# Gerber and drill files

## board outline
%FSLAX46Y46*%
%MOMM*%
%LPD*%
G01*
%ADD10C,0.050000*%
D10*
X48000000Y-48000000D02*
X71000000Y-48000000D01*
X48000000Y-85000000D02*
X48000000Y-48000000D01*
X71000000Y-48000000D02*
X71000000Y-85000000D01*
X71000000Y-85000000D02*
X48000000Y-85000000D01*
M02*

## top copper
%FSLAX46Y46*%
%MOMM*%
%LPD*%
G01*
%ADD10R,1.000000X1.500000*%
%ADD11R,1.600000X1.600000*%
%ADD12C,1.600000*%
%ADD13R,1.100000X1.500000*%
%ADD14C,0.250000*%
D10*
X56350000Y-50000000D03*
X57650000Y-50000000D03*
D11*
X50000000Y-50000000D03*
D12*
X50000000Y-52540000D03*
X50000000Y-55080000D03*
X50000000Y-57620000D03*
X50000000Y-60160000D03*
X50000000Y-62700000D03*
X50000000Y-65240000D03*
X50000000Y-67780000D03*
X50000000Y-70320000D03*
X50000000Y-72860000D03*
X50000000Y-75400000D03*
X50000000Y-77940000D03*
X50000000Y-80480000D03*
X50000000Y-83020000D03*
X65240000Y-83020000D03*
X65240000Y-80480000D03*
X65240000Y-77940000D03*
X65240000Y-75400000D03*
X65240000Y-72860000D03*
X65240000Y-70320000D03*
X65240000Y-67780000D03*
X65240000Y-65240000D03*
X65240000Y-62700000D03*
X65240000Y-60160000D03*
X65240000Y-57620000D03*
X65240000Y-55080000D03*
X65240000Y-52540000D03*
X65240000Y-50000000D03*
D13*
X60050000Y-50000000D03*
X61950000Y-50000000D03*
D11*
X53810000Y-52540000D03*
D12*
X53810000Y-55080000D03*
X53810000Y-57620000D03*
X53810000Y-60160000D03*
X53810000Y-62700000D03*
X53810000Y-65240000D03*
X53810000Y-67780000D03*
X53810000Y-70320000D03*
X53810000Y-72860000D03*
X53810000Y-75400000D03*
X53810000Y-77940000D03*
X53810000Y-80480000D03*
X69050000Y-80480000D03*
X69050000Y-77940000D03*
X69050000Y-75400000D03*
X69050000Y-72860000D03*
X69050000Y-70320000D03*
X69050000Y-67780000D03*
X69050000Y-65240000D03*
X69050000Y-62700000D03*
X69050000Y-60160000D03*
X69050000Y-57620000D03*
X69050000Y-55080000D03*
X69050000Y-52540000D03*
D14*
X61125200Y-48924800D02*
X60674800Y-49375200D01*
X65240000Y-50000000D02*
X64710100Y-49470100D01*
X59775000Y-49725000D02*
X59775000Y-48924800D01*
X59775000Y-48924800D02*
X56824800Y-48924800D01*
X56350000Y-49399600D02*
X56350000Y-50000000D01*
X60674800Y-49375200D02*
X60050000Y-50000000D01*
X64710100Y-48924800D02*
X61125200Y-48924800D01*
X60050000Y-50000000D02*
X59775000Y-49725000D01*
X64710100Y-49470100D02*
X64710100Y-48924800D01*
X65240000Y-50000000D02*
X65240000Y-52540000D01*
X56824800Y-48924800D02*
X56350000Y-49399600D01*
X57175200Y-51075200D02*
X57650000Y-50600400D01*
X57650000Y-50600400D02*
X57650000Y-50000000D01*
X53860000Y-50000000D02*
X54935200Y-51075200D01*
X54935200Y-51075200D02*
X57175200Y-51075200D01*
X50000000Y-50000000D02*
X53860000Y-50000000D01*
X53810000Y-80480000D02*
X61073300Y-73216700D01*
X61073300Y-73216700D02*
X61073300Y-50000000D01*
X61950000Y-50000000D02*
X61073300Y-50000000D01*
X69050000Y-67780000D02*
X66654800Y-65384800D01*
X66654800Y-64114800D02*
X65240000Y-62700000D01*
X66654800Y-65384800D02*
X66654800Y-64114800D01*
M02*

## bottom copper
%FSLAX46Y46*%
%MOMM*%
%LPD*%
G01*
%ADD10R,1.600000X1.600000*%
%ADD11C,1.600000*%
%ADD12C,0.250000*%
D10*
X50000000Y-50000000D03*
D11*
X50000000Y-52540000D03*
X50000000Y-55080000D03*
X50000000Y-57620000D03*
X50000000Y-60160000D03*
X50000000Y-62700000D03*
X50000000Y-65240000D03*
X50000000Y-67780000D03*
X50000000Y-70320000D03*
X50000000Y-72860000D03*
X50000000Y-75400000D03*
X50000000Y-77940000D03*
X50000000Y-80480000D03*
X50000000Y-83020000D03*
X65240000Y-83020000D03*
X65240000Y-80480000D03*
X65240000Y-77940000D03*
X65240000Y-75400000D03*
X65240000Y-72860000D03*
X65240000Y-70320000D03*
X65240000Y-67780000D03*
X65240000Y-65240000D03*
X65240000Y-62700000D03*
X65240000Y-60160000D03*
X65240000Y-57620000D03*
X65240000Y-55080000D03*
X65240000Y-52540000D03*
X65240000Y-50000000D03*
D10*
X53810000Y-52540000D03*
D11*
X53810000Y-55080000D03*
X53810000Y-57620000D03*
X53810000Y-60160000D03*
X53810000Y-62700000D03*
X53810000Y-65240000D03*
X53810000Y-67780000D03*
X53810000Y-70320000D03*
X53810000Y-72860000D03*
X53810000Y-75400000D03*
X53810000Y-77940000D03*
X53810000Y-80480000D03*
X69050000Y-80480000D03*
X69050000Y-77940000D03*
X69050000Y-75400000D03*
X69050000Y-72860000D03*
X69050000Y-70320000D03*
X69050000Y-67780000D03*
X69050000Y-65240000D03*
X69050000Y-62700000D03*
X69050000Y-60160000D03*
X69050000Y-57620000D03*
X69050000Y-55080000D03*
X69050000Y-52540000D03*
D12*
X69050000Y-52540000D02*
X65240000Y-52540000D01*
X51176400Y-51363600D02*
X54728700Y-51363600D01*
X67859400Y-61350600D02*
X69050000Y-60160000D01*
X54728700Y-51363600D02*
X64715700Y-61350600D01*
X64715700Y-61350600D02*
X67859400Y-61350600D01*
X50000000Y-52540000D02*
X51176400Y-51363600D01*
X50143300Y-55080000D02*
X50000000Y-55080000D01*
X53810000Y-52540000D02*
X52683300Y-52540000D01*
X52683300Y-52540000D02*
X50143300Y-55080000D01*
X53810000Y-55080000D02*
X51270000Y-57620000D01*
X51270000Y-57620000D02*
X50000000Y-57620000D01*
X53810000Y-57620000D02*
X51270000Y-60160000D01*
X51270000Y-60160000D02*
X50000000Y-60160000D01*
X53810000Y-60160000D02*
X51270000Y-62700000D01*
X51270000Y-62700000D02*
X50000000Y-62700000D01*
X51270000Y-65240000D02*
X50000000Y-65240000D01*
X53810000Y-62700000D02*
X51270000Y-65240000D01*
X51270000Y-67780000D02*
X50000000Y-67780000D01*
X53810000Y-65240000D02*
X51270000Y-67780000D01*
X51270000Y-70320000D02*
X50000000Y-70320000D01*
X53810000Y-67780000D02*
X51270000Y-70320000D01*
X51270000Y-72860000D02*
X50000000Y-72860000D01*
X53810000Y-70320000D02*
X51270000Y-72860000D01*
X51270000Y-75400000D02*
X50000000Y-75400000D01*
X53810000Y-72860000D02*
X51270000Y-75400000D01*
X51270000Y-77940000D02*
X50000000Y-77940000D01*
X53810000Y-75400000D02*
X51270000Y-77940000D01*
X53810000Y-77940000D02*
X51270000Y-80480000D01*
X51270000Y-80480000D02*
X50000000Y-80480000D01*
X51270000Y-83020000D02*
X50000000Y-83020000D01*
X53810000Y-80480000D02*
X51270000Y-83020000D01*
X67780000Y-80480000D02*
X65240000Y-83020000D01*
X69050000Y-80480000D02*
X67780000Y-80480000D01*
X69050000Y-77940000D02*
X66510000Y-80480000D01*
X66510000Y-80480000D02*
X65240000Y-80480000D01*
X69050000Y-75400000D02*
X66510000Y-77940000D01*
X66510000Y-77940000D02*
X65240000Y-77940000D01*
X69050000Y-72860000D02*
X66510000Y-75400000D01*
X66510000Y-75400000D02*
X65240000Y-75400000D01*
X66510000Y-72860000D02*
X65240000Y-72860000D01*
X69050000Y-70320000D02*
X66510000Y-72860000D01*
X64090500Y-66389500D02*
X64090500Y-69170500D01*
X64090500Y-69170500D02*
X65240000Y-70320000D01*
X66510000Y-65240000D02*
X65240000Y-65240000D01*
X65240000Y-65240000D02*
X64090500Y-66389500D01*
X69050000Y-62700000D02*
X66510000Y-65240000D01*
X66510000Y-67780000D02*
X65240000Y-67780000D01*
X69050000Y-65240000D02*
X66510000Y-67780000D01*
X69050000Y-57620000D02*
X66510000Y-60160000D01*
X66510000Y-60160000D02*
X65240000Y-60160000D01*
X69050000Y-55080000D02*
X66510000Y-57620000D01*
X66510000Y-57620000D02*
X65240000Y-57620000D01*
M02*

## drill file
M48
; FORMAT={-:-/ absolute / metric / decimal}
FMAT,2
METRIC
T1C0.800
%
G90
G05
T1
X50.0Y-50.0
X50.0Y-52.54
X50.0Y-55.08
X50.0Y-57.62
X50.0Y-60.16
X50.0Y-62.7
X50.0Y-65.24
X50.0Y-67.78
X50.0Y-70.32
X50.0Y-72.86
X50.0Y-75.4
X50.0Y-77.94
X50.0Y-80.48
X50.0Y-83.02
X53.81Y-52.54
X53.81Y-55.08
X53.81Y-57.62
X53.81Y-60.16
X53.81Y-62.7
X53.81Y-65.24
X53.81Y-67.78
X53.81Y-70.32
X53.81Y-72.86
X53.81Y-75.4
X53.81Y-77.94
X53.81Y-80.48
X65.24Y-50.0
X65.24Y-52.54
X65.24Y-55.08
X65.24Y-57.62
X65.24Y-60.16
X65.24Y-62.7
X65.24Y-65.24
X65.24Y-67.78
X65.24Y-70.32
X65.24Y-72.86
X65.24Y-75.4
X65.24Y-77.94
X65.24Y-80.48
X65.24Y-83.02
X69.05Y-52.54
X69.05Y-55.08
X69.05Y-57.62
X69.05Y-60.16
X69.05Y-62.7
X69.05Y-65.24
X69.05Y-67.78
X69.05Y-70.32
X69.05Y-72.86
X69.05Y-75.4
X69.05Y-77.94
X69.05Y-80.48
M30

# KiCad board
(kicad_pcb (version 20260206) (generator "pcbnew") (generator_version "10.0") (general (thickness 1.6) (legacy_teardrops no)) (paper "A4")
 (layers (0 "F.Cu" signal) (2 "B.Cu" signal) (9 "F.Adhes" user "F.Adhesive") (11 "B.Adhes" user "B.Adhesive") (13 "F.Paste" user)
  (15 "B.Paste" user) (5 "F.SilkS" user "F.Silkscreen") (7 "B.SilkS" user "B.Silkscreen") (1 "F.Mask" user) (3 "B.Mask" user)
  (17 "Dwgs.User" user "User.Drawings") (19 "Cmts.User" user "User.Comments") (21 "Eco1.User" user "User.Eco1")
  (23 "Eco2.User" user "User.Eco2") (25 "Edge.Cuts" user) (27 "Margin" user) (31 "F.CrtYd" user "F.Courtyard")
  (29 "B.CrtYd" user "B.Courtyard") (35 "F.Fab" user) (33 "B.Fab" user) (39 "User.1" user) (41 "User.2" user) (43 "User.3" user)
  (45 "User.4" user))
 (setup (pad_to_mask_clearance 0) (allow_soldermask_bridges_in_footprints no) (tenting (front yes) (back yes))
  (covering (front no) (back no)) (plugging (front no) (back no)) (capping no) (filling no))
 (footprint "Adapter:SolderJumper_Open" (layer "F.Cu") (at 57 50)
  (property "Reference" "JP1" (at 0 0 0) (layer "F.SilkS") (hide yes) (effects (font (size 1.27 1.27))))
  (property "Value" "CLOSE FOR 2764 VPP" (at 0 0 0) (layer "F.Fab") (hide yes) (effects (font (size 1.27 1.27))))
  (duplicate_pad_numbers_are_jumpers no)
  (pad "1" smd rect (at -0.65 0) (size 1 1.5) (layers "F.Cu" "F.Mask") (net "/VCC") (thermal_bridge_angle 45))
  (pad "2" smd rect (at 0.65 0) (size 1 1.5) (layers "F.Cu" "F.Mask") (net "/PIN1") (thermal_bridge_angle 45)))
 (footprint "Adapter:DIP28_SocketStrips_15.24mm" (layer "F.Cu") (at 50 50)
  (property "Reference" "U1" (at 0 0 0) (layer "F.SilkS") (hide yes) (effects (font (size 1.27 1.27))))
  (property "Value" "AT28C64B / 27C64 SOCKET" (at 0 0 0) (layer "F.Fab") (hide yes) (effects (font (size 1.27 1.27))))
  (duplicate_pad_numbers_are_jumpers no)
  (pad "1" thru_hole rect (at 0 0) (size 1.6 1.6) (drill 0.8) (layers "*.Cu" "*.Mask") (remove_unused_layers no) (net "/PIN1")
   (thermal_bridge_angle 45))
  (pad "2" thru_hole circle (at 0 2.54) (size 1.6 1.6) (drill 0.8) (layers "*.Cu" "*.Mask") (remove_unused_layers no) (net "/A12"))
  (pad "3" thru_hole circle (at 0 5.08) (size 1.6 1.6) (drill 0.8) (layers "*.Cu" "*.Mask") (remove_unused_layers no) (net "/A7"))
  (pad "4" thru_hole circle (at 0 7.62) (size 1.6 1.6) (drill 0.8) (layers "*.Cu" "*.Mask") (remove_unused_layers no) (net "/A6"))
  (pad "5" thru_hole circle (at 0 10.16) (size 1.6 1.6) (drill 0.8) (layers "*.Cu" "*.Mask") (remove_unused_layers no) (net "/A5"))
  (pad "6" thru_hole circle (at 0 12.7) (size 1.6 1.6) (drill 0.8) (layers "*.Cu" "*.Mask") (remove_unused_layers no) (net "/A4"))
  (pad "7" thru_hole circle (at 0 15.24) (size 1.6 1.6) (drill 0.8) (layers "*.Cu" "*.Mask") (remove_unused_layers no) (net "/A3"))
  (pad "8" thru_hole circle (at 0 17.78) (size 1.6 1.6) (drill 0.8) (layers "*.Cu" "*.Mask") (remove_unused_layers no) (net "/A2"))
  (pad "9" thru_hole circle (at 0 20.32) (size 1.6 1.6) (drill 0.8) (layers "*.Cu" "*.Mask") (remove_unused_layers no) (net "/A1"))
  (pad "10" thru_hole circle (at 0 22.86) (size 1.6 1.6) (drill 0.8) (layers "*.Cu" "*.Mask") (remove_unused_layers no) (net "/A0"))
  (pad "11" thru_hole circle (at 0 25.4) (size 1.6 1.6) (drill 0.8) (layers "*.Cu" "*.Mask") (remove_unused_layers no) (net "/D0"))
  (pad "12" thru_hole circle (at 0 27.94) (size 1.6 1.6) (drill 0.8) (layers "*.Cu" "*.Mask") (remove_unused_layers no) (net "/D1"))
  (pad "13" thru_hole circle (at 0 30.48) (size 1.6 1.6) (drill 0.8) (layers "*.Cu" "*.Mask") (remove_unused_layers no) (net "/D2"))
  (pad "14" thru_hole circle (at 0 33.02) (size 1.6 1.6) (drill 0.8) (layers "*.Cu" "*.Mask") (remove_unused_layers no) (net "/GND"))
  (pad "15" thru_hole circle (at 15.24 33.02) (size 1.6 1.6) (drill 0.8) (layers "*.Cu" "*.Mask") (remove_unused_layers no) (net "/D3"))
  (pad "16" thru_hole circle (at 15.24 30.48) (size 1.6 1.6) (drill 0.8) (layers "*.Cu" "*.Mask") (remove_unused_layers no) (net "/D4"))
  (pad "17" thru_hole circle (at 15.24 27.94) (size 1.6 1.6) (drill 0.8) (layers "*.Cu" "*.Mask") (remove_unused_layers no) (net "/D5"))
  (pad "18" thru_hole circle (at 15.24 25.4) (size 1.6 1.6) (drill 0.8) (layers "*.Cu" "*.Mask") (remove_unused_layers no) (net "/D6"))
  (pad "19" thru_hole circle (at 15.24 22.86) (size 1.6 1.6) (drill 0.8) (layers "*.Cu" "*.Mask") (remove_unused_layers no) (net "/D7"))
  (pad "20" thru_hole circle (at 15.24 20.32) (size 1.6 1.6) (drill 0.8) (layers "*.Cu" "*.Mask") (remove_unused_layers no)
   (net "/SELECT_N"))
  (pad "21" thru_hole circle (at 15.24 17.78) (size 1.6 1.6) (drill 0.8) (layers "*.Cu" "*.Mask") (remove_unused_layers no) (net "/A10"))
  (pad "22" thru_hole circle (at 15.24 15.24) (size 1.6 1.6) (drill 0.8) (layers "*.Cu" "*.Mask") (remove_unused_layers no)
   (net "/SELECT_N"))
  (pad "23" thru_hole circle (at 15.24 12.7) (size 1.6 1.6) (drill 0.8) (layers "*.Cu" "*.Mask") (remove_unused_layers no) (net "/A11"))
  (pad "24" thru_hole circle (at 15.24 10.16) (size 1.6 1.6) (drill 0.8) (layers "*.Cu" "*.Mask") (remove_unused_layers no) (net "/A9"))
  (pad "25" thru_hole circle (at 15.24 7.62) (size 1.6 1.6) (drill 0.8) (layers "*.Cu" "*.Mask") (remove_unused_layers no) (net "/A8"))
  (pad "26" thru_hole circle (at 15.24 5.08) (size 1.6 1.6) (drill 0.8) (layers "*.Cu" "*.Mask") (remove_unused_layers no)
   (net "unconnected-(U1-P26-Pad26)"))
  (pad "27" thru_hole circle (at 15.24 2.54) (size 1.6 1.6) (drill 0.8) (layers "*.Cu" "*.Mask") (remove_unused_layers no) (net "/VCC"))
  (pad "28" thru_hole circle (at 15.24 0) (size 1.6 1.6) (drill 0.8) (layers "*.Cu" "*.Mask") (remove_unused_layers no) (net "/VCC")))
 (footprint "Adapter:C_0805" (layer "F.Cu") (at 61 50)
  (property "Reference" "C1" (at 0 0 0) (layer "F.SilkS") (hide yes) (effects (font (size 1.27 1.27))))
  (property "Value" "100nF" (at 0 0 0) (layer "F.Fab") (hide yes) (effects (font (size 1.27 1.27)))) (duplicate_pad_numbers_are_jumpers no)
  (pad "1" smd rect (at -0.95 0) (size 1.1 1.5) (layers "F.Cu" "F.Mask" "F.Paste") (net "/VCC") (thermal_bridge_angle 45))
  (pad "2" smd rect (at 0.95 0) (size 1.1 1.5) (layers "F.Cu" "F.Mask" "F.Paste") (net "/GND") (thermal_bridge_angle 45)))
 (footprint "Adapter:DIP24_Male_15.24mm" (layer "B.Cu") (at 53.81 52.54)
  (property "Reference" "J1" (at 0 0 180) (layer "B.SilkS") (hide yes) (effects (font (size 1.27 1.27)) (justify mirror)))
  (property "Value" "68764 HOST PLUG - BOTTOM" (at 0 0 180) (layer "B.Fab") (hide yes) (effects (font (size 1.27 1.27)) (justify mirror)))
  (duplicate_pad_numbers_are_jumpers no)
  (pad "1" thru_hole rect (at 0 0) (size 1.6 1.6) (drill 0.8) (layers "*.Cu" "*.Mask") (remove_unused_layers no) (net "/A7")
   (thermal_bridge_angle 45))
  (pad "2" thru_hole circle (at 0 2.54) (size 1.6 1.6) (drill 0.8) (layers "*.Cu" "*.Mask") (remove_unused_layers no) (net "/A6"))
  (pad "3" thru_hole circle (at 0 5.08) (size 1.6 1.6) (drill 0.8) (layers "*.Cu" "*.Mask") (remove_unused_layers no) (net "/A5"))
  (pad "4" thru_hole circle (at 0 7.62) (size 1.6 1.6) (drill 0.8) (layers "*.Cu" "*.Mask") (remove_unused_layers no) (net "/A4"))
  (pad "5" thru_hole circle (at 0 10.16) (size 1.6 1.6) (drill 0.8) (layers "*.Cu" "*.Mask") (remove_unused_layers no) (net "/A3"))
  (pad "6" thru_hole circle (at 0 12.7) (size 1.6 1.6) (drill 0.8) (layers "*.Cu" "*.Mask") (remove_unused_layers no) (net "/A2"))
  (pad "7" thru_hole circle (at 0 15.24) (size 1.6 1.6) (drill 0.8) (layers "*.Cu" "*.Mask") (remove_unused_layers no) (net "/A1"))
  (pad "8" thru_hole circle (at 0 17.78) (size 1.6 1.6) (drill 0.8) (layers "*.Cu" "*.Mask") (remove_unused_layers no) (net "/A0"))
  (pad "9" thru_hole circle (at 0 20.32) (size 1.6 1.6) (drill 0.8) (layers "*.Cu" "*.Mask") (remove_unused_layers no) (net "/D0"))
  (pad "10" thru_hole circle (at 0 22.86) (size 1.6 1.6) (drill 0.8) (layers "*.Cu" "*.Mask") (remove_unused_layers no) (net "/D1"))
  (pad "11" thru_hole circle (at 0 25.4) (size 1.6 1.6) (drill 0.8) (layers "*.Cu" "*.Mask") (remove_unused_layers no) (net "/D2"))
  (pad "12" thru_hole circle (at 0 27.94) (size 1.6 1.6) (drill 0.8) (layers "*.Cu" "*.Mask") (remove_unused_layers no) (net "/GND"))
  (pad "13" thru_hole circle (at 15.24 27.94) (size 1.6 1.6) (drill 0.8) (layers "*.Cu" "*.Mask") (remove_unused_layers no) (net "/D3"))
  (pad "14" thru_hole circle (at 15.24 25.4) (size 1.6 1.6) (drill 0.8) (layers "*.Cu" "*.Mask") (remove_unused_layers no) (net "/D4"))
  (pad "15" thru_hole circle (at 15.24 22.86) (size 1.6 1.6) (drill 0.8) (layers "*.Cu" "*.Mask") (remove_unused_layers no) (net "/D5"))
  (pad "16" thru_hole circle (at 15.24 20.32) (size 1.6 1.6) (drill 0.8) (layers "*.Cu" "*.Mask") (remove_unused_layers no) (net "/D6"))
  (pad "17" thru_hole circle (at 15.24 17.78) (size 1.6 1.6) (drill 0.8) (layers "*.Cu" "*.Mask") (remove_unused_layers no) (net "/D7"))
  (pad "18" thru_hole circle (at 15.24 15.24) (size 1.6 1.6) (drill 0.8) (layers "*.Cu" "*.Mask") (remove_unused_layers no) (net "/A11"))
  (pad "19" thru_hole circle (at 15.24 12.7) (size 1.6 1.6) (drill 0.8) (layers "*.Cu" "*.Mask") (remove_unused_layers no) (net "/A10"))
  (pad "20" thru_hole circle (at 15.24 10.16) (size 1.6 1.6) (drill 0.8) (layers "*.Cu" "*.Mask") (remove_unused_layers no)
   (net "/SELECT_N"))
  (pad "21" thru_hole circle (at 15.24 7.62) (size 1.6 1.6) (drill 0.8) (layers "*.Cu" "*.Mask") (remove_unused_layers no) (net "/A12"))
  (pad "22" thru_hole circle (at 15.24 5.08) (size 1.6 1.6) (drill 0.8) (layers "*.Cu" "*.Mask") (remove_unused_layers no) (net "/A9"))
  (pad "23" thru_hole circle (at 15.24 2.54) (size 1.6 1.6) (drill 0.8) (layers "*.Cu" "*.Mask") (remove_unused_layers no) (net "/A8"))
  (pad "24" thru_hole circle (at 15.24 0) (size 1.6 1.6) (drill 0.8) (layers "*.Cu" "*.Mask") (remove_unused_layers no) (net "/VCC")))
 (gr_line (start 48 48) (end 71 48) (stroke (width 0.05) (type default)) (layer "Edge.Cuts"))
 (gr_line (start 48 85) (end 48 48) (stroke (width 0.05) (type default)) (layer "Edge.Cuts"))
 (gr_line (start 71 48) (end 71 85) (stroke (width 0.05) (type default)) (layer "Edge.Cuts"))
 (gr_line (start 71 85) (end 48 85) (stroke (width 0.05) (type default)) (layer "Edge.Cuts"))
 (segment (start 61.1252 48.9248) (end 60.6748 49.3752) (width 0.25) (layer "F.Cu") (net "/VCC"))
 (segment (start 65.24 50) (end 64.7101 49.4701) (width 0.25) (layer "F.Cu") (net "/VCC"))
 (segment (start 59.775 49.725) (end 59.775 48.9248) (width 0.25) (layer "F.Cu") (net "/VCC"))
 (segment (start 59.775 48.9248) (end 56.8248 48.9248) (width 0.25) (layer "F.Cu") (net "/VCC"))
 (segment (start 56.35 49.3996) (end 56.35 50) (width 0.25) (layer "F.Cu") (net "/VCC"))
 (segment (start 60.6748 49.3752) (end 60.05 50) (width 0.25) (layer "F.Cu") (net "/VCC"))
 (segment (start 64.7101 48.9248) (end 61.1252 48.9248) (width 0.25) (layer "F.Cu") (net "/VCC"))
 (segment (start 60.05 50) (end 59.775 49.725) (width 0.25) (layer "F.Cu") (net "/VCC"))
 (segment (start 64.7101 49.4701) (end 64.7101 48.9248) (width 0.25) (layer "F.Cu") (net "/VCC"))
 (segment (start 65.24 50) (end 65.24 52.54) (width 0.25) (layer "F.Cu") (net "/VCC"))
 (segment (start 56.8248 48.9248) (end 56.35 49.3996) (width 0.25) (layer "F.Cu") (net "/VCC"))
 (segment (start 69.05 52.54) (end 65.24 52.54) (width 0.25) (layer "B.Cu") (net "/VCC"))
 (segment (start 57.1752 51.0752) (end 57.65 50.6004) (width 0.25) (layer "F.Cu") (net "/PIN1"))
 (segment (start 57.65 50.6004) (end 57.65 50) (width 0.25) (layer "F.Cu") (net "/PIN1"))
 (segment (start 53.86 50) (end 54.9352 51.0752) (width 0.25) (layer "F.Cu") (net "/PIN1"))
 (segment (start 54.9352 51.0752) (end 57.1752 51.0752) (width 0.25) (layer "F.Cu") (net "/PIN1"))
 (segment (start 50 50) (end 53.86 50) (width 0.25) (layer "F.Cu") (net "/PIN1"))
 (segment (start 51.1764 51.3636) (end 54.7287 51.3636) (width 0.25) (layer "B.Cu") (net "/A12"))
 (segment (start 67.8594 61.3506) (end 69.05 60.16) (width 0.25) (layer "B.Cu") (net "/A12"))
 (segment (start 54.7287 51.3636) (end 64.7157 61.3506) (width 0.25) (layer "B.Cu") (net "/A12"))
 (segment (start 64.7157 61.3506) (end 67.8594 61.3506) (width 0.25) (layer "B.Cu") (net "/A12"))
 (segment (start 50 52.54) (end 51.1764 51.3636) (width 0.25) (layer "B.Cu") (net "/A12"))
 (segment (start 50.1433 55.08) (end 50 55.08) (width 0.25) (layer "B.Cu") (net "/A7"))
 (segment (start 53.81 52.54) (end 52.6833 52.54) (width 0.25) (layer "B.Cu") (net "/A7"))
 (segment (start 52.6833 52.54) (end 50.1433 55.08) (width 0.25) (layer "B.Cu") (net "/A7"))
 (segment (start 53.81 55.08) (end 51.27 57.62) (width 0.25) (layer "B.Cu") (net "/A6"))
 (segment (start 51.27 57.62) (end 50 57.62) (width 0.25) (layer "B.Cu") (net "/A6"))
 (segment (start 53.81 57.62) (end 51.27 60.16) (width 0.25) (layer "B.Cu") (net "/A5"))
 (segment (start 51.27 60.16) (end 50 60.16) (width 0.25) (layer "B.Cu") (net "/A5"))
 (segment (start 53.81 60.16) (end 51.27 62.7) (width 0.25) (layer "B.Cu") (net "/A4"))
 (segment (start 51.27 62.7) (end 50 62.7) (width 0.25) (layer "B.Cu") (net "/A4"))
 (segment (start 51.27 65.24) (end 50 65.24) (width 0.25) (layer "B.Cu") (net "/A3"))
 (segment (start 53.81 62.7) (end 51.27 65.24) (width 0.25) (layer "B.Cu") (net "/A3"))
 (segment (start 51.27 67.78) (end 50 67.78) (width 0.25) (layer "B.Cu") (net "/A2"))
 (segment (start 53.81 65.24) (end 51.27 67.78) (width 0.25) (layer "B.Cu") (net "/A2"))
 (segment (start 51.27 70.32) (end 50 70.32) (width 0.25) (layer "B.Cu") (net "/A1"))
 (segment (start 53.81 67.78) (end 51.27 70.32) (width 0.25) (layer "B.Cu") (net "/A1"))
 (segment (start 51.27 72.86) (end 50 72.86) (width 0.25) (layer "B.Cu") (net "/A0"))
 (segment (start 53.81 70.32) (end 51.27 72.86) (width 0.25) (layer "B.Cu") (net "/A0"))
 (segment (start 51.27 75.4) (end 50 75.4) (width 0.25) (layer "B.Cu") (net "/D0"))
 (segment (start 53.81 72.86) (end 51.27 75.4) (width 0.25) (layer "B.Cu") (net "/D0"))
 (segment (start 51.27 77.94) (end 50 77.94) (width 0.25) (layer "B.Cu") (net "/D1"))
 (segment (start 53.81 75.4) (end 51.27 77.94) (width 0.25) (layer "B.Cu") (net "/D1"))
 (segment (start 53.81 77.94) (end 51.27 80.48) (width 0.25) (layer "B.Cu") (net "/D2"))
 (segment (start 51.27 80.48) (end 50 80.48) (width 0.25) (layer "B.Cu") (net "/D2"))
 (segment (start 53.81 80.48) (end 61.0733 73.2167) (width 0.25) (layer "F.Cu") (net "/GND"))
 (segment (start 61.0733 73.2167) (end 61.0733 50) (width 0.25) (layer "F.Cu") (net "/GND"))
 (segment (start 61.95 50) (end 61.0733 50) (width 0.25) (layer "F.Cu") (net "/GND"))
 (segment (start 51.27 83.02) (end 50 83.02) (width 0.25) (layer "B.Cu") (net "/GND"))
 (segment (start 53.81 80.48) (end 51.27 83.02) (width 0.25) (layer "B.Cu") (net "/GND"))
 (segment (start 67.78 80.48) (end 65.24 83.02) (width 0.25) (layer "B.Cu") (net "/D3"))
 (segment (start 69.05 80.48) (end 67.78 80.48) (width 0.25) (layer "B.Cu") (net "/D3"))
 (segment (start 69.05 77.94) (end 66.51 80.48) (width 0.25) (layer "B.Cu") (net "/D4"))
 (segment (start 66.51 80.48) (end 65.24 80.48) (width 0.25) (layer "B.Cu") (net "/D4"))
 (segment (start 69.05 75.4) (end 66.51 77.94) (width 0.25) (layer "B.Cu") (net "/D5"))
 (segment (start 66.51 77.94) (end 65.24 77.94) (width 0.25) (layer "B.Cu") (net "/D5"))
 (segment (start 69.05 72.86) (end 66.51 75.4) (width 0.25) (layer "B.Cu") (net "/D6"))
 (segment (start 66.51 75.4) (end 65.24 75.4) (width 0.25) (layer "B.Cu") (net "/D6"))
 (segment (start 66.51 72.86) (end 65.24 72.86) (width 0.25) (layer "B.Cu") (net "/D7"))
 (segment (start 69.05 70.32) (end 66.51 72.86) (width 0.25) (layer "B.Cu") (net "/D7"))
 (segment (start 64.0905 66.3895) (end 64.0905 69.1705) (width 0.25) (layer "B.Cu") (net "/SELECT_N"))
 (segment (start 64.0905 69.1705) (end 65.24 70.32) (width 0.25) (layer "B.Cu") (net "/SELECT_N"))
 (segment (start 66.51 65.24) (end 65.24 65.24) (width 0.25) (layer "B.Cu") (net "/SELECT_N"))
 (segment (start 65.24 65.24) (end 64.0905 66.3895) (width 0.25) (layer "B.Cu") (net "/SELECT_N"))
 (segment (start 69.05 62.7) (end 66.51 65.24) (width 0.25) (layer "B.Cu") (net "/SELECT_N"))
 (segment (start 66.51 67.78) (end 65.24 67.78) (width 0.25) (layer "B.Cu") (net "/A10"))
 (segment (start 69.05 65.24) (end 66.51 67.78) (width 0.25) (layer "B.Cu") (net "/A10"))
 (segment (start 69.05 67.78) (end 66.6548 65.3848) (width 0.25) (layer "F.Cu") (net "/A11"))
 (segment (start 66.6548 64.1148) (end 65.24 62.7) (width 0.25) (layer "F.Cu") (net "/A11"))
 (segment (start 66.6548 65.3848) (end 66.6548 64.1148) (width 0.25) (layer "F.Cu") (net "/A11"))
 (segment (start 69.05 57.62) (end 66.51 60.16) (width 0.25) (layer "B.Cu") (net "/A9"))
 (segment (start 66.51 60.16) (end 65.24 60.16) (width 0.25) (layer "B.Cu") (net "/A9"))
 (segment (start 69.05 55.08) (end 66.51 57.62) (width 0.25) (layer "B.Cu") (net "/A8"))
 (segment (start 66.51 57.62) (end 65.24 57.62) (width 0.25) (layer "B.Cu") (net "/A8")))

